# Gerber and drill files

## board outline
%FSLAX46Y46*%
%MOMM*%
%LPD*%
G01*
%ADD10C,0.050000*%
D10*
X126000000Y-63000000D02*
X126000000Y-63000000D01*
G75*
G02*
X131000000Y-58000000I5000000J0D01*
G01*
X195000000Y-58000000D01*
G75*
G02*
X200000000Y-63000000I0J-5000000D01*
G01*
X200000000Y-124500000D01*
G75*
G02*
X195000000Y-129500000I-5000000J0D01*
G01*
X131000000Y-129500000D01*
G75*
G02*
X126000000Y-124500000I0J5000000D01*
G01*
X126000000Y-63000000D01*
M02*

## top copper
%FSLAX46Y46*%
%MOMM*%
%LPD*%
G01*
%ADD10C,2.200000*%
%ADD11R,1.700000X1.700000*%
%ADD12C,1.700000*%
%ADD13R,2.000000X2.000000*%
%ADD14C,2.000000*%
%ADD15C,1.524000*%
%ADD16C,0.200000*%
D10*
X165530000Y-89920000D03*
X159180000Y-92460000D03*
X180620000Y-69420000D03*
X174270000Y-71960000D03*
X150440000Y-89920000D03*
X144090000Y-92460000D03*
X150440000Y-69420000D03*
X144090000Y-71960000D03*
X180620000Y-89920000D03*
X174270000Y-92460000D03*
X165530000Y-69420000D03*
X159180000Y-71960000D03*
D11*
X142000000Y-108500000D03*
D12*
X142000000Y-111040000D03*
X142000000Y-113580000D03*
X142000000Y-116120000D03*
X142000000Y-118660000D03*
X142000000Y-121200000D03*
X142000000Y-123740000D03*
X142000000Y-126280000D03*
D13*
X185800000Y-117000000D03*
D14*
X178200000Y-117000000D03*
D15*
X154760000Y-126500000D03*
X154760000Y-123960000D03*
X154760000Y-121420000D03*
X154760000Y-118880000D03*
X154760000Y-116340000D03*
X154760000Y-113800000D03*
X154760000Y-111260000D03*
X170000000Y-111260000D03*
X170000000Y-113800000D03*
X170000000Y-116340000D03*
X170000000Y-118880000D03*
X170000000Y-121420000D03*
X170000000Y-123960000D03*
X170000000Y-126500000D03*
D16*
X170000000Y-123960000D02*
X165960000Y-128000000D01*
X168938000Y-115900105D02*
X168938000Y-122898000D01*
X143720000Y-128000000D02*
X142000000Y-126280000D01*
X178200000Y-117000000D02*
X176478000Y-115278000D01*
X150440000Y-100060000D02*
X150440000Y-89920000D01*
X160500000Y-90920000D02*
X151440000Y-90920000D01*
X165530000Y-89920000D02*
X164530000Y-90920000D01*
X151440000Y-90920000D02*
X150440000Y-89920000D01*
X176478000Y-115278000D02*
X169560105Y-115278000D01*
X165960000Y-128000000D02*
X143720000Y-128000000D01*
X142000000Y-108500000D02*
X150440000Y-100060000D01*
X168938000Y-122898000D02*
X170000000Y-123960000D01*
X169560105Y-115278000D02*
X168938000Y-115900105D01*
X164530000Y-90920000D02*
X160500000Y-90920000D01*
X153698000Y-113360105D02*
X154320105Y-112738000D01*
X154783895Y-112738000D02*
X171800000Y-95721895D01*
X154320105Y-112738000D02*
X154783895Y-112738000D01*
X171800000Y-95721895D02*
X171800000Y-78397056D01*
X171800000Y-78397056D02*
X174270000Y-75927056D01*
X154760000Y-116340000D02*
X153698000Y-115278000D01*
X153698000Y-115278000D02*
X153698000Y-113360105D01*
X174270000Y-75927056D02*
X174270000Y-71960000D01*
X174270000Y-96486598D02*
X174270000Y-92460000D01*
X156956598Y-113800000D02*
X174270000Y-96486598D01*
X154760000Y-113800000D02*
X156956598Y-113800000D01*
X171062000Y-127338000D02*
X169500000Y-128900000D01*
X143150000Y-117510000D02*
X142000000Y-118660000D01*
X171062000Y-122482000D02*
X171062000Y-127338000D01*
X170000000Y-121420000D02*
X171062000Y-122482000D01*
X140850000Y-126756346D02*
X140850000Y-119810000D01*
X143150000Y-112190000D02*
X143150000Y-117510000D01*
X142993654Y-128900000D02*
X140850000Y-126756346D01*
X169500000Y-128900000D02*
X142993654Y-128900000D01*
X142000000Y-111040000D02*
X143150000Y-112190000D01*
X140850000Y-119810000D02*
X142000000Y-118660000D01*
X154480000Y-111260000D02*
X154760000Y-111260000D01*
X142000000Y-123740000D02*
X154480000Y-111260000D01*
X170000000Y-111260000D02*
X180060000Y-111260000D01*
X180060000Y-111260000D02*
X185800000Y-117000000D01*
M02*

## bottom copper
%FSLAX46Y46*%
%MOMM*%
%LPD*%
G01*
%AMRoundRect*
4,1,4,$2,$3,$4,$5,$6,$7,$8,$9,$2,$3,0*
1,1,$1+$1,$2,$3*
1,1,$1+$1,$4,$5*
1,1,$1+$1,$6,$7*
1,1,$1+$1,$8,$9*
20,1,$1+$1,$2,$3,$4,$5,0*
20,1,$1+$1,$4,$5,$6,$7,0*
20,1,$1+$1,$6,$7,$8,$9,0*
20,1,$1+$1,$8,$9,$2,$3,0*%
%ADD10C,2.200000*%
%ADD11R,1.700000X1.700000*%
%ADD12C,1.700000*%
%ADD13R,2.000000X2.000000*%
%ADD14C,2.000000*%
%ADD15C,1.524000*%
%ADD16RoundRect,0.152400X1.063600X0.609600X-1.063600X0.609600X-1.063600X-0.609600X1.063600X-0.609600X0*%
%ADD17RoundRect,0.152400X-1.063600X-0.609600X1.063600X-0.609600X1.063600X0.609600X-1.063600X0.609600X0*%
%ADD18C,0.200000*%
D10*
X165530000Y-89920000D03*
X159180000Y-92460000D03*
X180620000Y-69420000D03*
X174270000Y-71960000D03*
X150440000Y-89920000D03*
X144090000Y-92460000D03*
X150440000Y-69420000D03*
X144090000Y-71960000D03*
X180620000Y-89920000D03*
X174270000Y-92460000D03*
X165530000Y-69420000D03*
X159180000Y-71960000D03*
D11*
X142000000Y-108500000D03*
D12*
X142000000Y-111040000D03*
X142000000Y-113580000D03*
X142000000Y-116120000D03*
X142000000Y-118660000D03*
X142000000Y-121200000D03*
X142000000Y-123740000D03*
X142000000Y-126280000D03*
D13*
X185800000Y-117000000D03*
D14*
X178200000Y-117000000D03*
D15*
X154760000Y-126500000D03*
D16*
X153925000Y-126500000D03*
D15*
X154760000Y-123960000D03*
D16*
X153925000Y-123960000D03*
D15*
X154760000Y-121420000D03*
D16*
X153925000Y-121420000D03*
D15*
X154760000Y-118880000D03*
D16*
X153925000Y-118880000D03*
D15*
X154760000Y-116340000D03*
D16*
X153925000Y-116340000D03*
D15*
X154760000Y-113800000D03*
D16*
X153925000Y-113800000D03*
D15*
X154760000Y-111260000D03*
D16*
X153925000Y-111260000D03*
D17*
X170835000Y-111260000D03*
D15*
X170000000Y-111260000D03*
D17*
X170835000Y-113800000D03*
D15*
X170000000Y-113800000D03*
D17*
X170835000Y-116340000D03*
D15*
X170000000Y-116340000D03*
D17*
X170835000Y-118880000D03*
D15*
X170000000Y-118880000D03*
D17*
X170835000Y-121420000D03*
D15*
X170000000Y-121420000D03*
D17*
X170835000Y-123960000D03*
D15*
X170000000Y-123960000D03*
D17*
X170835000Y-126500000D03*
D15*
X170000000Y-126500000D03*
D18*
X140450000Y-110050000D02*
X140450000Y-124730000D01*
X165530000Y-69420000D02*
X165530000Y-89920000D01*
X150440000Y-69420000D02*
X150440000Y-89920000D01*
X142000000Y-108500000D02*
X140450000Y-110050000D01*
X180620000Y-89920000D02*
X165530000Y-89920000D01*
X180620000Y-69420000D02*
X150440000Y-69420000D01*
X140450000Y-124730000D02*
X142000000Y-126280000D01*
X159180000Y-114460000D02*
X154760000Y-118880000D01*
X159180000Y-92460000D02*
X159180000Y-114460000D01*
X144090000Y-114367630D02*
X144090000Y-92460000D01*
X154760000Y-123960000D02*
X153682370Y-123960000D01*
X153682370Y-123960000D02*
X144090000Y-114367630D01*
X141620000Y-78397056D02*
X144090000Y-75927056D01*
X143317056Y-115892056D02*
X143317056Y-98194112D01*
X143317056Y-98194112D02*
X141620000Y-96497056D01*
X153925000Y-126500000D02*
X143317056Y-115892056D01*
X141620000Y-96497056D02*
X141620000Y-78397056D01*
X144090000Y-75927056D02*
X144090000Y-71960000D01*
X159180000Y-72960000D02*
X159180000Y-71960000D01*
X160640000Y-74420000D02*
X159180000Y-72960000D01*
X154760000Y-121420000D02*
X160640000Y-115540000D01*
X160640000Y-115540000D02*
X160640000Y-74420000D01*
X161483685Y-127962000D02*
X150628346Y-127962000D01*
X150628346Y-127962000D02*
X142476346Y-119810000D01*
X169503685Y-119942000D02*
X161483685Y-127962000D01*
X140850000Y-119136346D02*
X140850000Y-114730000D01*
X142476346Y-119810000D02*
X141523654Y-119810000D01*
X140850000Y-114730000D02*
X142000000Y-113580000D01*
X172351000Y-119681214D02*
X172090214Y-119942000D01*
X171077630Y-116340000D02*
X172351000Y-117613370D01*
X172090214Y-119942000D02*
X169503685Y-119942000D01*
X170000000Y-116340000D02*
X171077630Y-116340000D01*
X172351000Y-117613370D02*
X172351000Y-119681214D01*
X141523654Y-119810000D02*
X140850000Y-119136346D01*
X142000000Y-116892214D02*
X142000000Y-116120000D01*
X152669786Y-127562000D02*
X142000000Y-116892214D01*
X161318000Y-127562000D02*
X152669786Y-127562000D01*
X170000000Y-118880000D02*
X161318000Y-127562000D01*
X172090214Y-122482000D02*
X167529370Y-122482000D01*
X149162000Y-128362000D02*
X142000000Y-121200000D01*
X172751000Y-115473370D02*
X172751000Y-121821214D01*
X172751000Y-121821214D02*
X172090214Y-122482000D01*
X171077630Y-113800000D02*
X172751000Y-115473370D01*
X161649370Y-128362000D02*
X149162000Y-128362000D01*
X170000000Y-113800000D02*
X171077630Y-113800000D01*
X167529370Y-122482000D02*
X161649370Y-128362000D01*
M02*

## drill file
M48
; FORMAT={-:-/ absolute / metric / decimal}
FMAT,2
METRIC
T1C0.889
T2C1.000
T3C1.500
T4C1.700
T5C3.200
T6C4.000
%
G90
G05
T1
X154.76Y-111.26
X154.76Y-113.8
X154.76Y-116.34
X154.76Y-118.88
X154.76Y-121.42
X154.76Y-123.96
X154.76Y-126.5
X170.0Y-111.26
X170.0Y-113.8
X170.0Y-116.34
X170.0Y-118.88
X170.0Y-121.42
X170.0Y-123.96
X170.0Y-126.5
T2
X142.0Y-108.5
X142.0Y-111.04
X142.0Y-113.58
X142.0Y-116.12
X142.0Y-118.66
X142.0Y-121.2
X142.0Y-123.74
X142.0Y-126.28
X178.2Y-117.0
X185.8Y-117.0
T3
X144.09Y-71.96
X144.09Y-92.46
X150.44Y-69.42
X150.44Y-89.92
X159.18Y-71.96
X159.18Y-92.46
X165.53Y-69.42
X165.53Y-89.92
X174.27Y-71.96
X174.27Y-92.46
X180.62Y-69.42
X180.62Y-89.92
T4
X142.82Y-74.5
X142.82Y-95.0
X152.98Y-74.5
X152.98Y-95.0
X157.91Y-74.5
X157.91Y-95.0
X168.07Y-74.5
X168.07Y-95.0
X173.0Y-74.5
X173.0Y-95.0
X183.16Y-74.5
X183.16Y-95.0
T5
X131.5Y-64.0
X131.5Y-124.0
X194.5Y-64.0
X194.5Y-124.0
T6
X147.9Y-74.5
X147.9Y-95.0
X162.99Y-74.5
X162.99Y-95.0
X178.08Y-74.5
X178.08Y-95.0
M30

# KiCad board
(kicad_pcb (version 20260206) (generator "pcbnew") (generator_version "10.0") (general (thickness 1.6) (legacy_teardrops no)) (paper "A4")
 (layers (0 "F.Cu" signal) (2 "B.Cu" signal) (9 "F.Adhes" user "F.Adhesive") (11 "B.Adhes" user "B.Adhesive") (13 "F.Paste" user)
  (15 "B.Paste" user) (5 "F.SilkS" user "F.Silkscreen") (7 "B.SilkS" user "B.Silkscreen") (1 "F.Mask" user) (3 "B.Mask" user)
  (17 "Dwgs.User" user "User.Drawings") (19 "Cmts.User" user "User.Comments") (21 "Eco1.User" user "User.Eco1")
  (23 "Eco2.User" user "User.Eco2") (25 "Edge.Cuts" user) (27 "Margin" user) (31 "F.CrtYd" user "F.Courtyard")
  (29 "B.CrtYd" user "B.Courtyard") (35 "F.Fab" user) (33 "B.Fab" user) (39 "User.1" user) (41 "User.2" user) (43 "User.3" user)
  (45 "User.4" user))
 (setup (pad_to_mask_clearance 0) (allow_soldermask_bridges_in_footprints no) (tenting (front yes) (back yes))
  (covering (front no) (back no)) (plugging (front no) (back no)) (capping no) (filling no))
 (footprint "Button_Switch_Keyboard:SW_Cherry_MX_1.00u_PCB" (layer "F.Cu") (at 165.53 89.92)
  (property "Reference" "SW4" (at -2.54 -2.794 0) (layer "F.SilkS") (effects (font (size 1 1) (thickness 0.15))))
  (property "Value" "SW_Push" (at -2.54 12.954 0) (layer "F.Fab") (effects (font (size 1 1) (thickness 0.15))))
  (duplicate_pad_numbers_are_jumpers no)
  (pad "" np_thru_hole circle (at -7.62 5.08) (size 1.7 1.7) (drill 1.7) (layers "*.Cu" "*.Mask"))
  (pad "" np_thru_hole circle (at -2.54 5.08) (size 4 4) (drill 4) (layers "*.Cu" "*.Mask"))
  (pad "" np_thru_hole circle (at 2.54 5.08) (size 1.7 1.7) (drill 1.7) (layers "*.Cu" "*.Mask"))
  (pad "1" thru_hole circle (at 0 0) (size 2.2 2.2) (drill 1.5) (layers "*.Cu" "*.Mask") (remove_unused_layers no) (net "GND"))
  (pad "2" thru_hole circle (at -6.35 2.54) (size 2.2 2.2) (drill 1.5) (layers "*.Cu" "*.Mask") (remove_unused_layers no)
   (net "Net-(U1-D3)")))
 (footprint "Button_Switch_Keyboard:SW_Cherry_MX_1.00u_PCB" (layer "F.Cu") (at 180.62 69.42)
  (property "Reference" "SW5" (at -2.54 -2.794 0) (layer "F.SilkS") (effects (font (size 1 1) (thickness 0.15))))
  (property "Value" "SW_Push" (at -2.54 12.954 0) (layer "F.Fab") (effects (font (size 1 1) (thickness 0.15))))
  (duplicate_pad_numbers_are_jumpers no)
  (pad "" np_thru_hole circle (at -7.62 5.08) (size 1.7 1.7) (drill 1.7) (layers "*.Cu" "*.Mask"))
  (pad "" np_thru_hole circle (at -2.54 5.08) (size 4 4) (drill 4) (layers "*.Cu" "*.Mask"))
  (pad "" np_thru_hole circle (at 2.54 5.08) (size 1.7 1.7) (drill 1.7) (layers "*.Cu" "*.Mask"))
  (pad "1" thru_hole circle (at 0 0) (size 2.2 2.2) (drill 1.5) (layers "*.Cu" "*.Mask") (remove_unused_layers no) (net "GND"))
  (pad "2" thru_hole circle (at -6.35 2.54) (size 2.2 2.2) (drill 1.5) (layers "*.Cu" "*.Mask") (remove_unused_layers no)
   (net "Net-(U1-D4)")))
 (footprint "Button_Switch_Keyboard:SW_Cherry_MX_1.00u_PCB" (layer "F.Cu") (at 150.44 89.92)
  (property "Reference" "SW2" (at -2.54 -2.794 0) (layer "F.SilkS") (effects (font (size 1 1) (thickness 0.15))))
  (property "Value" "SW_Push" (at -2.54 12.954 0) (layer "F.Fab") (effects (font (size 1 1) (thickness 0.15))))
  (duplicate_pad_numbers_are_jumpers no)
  (pad "" np_thru_hole circle (at -7.62 5.08) (size 1.7 1.7) (drill 1.7) (layers "*.Cu" "*.Mask"))
  (pad "" np_thru_hole circle (at -2.54 5.08) (size 4 4) (drill 4) (layers "*.Cu" "*.Mask"))
  (pad "" np_thru_hole circle (at 2.54 5.08) (size 1.7 1.7) (drill 1.7) (layers "*.Cu" "*.Mask"))
  (pad "1" thru_hole circle (at 0 0) (size 2.2 2.2) (drill 1.5) (layers "*.Cu" "*.Mask") (remove_unused_layers no) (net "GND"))
  (pad "2" thru_hole circle (at -6.35 2.54) (size 2.2 2.2) (drill 1.5) (layers "*.Cu" "*.Mask") (remove_unused_layers no)
   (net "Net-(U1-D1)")))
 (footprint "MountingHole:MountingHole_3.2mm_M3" (layer "F.Cu") (at 131.5 64)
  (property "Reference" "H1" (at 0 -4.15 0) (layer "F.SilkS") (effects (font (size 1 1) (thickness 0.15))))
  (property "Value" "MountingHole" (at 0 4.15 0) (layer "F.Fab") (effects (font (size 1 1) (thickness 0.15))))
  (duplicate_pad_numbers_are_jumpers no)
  (pad "" np_thru_hole circle (at 0 0) (size 3.2 3.2) (drill 3.2) (layers "*.Cu" "*.Mask")))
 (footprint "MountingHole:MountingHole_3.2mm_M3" (layer "F.Cu") (at 194.5 64)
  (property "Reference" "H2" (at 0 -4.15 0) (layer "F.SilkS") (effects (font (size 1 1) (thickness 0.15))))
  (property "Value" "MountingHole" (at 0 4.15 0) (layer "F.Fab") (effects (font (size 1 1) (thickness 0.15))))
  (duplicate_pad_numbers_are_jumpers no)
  (pad "" np_thru_hole circle (at 0 0) (size 3.2 3.2) (drill 3.2) (layers "*.Cu" "*.Mask")))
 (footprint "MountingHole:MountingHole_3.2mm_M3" (layer "F.Cu") (at 131.5 124)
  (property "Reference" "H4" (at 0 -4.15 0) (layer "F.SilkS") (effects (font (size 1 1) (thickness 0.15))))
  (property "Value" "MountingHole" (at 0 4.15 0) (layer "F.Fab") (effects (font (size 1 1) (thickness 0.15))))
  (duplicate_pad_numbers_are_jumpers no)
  (pad "" np_thru_hole circle (at 0 0) (size 3.2 3.2) (drill 3.2) (layers "*.Cu" "*.Mask")))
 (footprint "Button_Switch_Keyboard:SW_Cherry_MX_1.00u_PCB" (layer "F.Cu") (at 150.44 69.42)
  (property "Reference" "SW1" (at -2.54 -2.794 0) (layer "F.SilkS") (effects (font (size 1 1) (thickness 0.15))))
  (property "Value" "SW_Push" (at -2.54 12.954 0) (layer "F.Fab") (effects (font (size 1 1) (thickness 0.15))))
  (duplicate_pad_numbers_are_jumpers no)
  (pad "" np_thru_hole circle (at -7.62 5.08) (size 1.7 1.7) (drill 1.7) (layers "*.Cu" "*.Mask"))
  (pad "" np_thru_hole circle (at -2.54 5.08) (size 4 4) (drill 4) (layers "*.Cu" "*.Mask"))
  (pad "" np_thru_hole circle (at 2.54 5.08) (size 1.7 1.7) (drill 1.7) (layers "*.Cu" "*.Mask"))
  (pad "1" thru_hole circle (at 0 0) (size 2.2 2.2) (drill 1.5) (layers "*.Cu" "*.Mask") (remove_unused_layers no) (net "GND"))
  (pad "2" thru_hole circle (at -6.35 2.54) (size 2.2 2.2) (drill 1.5) (layers "*.Cu" "*.Mask") (remove_unused_layers no)
   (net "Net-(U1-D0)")))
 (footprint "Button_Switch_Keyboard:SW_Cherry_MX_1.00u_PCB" (layer "F.Cu") (at 180.62 89.92)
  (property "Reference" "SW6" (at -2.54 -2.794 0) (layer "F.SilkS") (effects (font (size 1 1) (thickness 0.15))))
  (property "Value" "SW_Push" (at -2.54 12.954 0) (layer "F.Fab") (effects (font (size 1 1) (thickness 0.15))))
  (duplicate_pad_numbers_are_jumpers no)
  (pad "" np_thru_hole circle (at -7.62 5.08) (size 1.7 1.7) (drill 1.7) (layers "*.Cu" "*.Mask"))
  (pad "" np_thru_hole circle (at -2.54 5.08) (size 4 4) (drill 4) (layers "*.Cu" "*.Mask"))
  (pad "" np_thru_hole circle (at 2.54 5.08) (size 1.7 1.7) (drill 1.7) (layers "*.Cu" "*.Mask"))
  (pad "1" thru_hole circle (at 0 0) (size 2.2 2.2) (drill 1.5) (layers "*.Cu" "*.Mask") (remove_unused_layers no) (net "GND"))
  (pad "2" thru_hole circle (at -6.35 2.54) (size 2.2 2.2) (drill 1.5) (layers "*.Cu" "*.Mask") (remove_unused_layers no)
   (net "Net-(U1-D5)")))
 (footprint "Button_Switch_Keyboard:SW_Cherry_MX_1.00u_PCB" (layer "F.Cu") (at 165.53 69.42)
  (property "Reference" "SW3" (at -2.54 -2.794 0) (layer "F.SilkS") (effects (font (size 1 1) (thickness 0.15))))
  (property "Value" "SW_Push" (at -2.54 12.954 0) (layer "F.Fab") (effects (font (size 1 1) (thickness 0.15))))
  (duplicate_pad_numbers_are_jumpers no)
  (pad "" np_thru_hole circle (at -7.62 5.08) (size 1.7 1.7) (drill 1.7) (layers "*.Cu" "*.Mask"))
  (pad "" np_thru_hole circle (at -2.54 5.08) (size 4 4) (drill 4) (layers "*.Cu" "*.Mask"))
  (pad "" np_thru_hole circle (at 2.54 5.08) (size 1.7 1.7) (drill 1.7) (layers "*.Cu" "*.Mask"))
  (pad "1" thru_hole circle (at 0 0) (size 2.2 2.2) (drill 1.5) (layers "*.Cu" "*.Mask") (remove_unused_layers no) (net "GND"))
  (pad "2" thru_hole circle (at -6.35 2.54) (size 2.2 2.2) (drill 1.5) (layers "*.Cu" "*.Mask") (remove_unused_layers no)
   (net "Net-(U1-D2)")))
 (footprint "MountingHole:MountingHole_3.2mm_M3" (layer "F.Cu") (at 194.5 124)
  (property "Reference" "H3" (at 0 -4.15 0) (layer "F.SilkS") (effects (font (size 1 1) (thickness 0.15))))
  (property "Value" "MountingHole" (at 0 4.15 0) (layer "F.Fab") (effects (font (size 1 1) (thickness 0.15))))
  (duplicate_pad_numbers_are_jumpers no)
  (pad "" np_thru_hole circle (at 0 0) (size 3.2 3.2) (drill 3.2) (layers "*.Cu" "*.Mask")))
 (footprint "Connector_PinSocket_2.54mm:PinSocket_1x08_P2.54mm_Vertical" (layer "B.Cu") (at 142 108.5 180)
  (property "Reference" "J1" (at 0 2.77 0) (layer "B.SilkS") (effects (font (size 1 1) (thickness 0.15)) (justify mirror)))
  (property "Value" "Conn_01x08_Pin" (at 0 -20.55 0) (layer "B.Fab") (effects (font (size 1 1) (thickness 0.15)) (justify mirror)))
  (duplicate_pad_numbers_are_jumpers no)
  (pad "1" thru_hole rect (at 0 0 180) (size 1.7 1.7) (drill 1) (layers "*.Cu" "*.Mask") (remove_unused_layers no) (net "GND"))
  (pad "2" thru_hole circle (at 0 -2.54 180) (size 1.7 1.7) (drill 1) (layers "*.Cu" "*.Mask") (remove_unused_layers no) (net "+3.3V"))
  (pad "3" thru_hole circle (at 0 -5.08 180) (size 1.7 1.7) (drill 1) (layers "*.Cu" "*.Mask") (remove_unused_layers no) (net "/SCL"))
  (pad "4" thru_hole circle (at 0 -7.62 180) (size 1.7 1.7) (drill 1) (layers "*.Cu" "*.Mask") (remove_unused_layers no) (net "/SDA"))
  (pad "5" thru_hole circle (at 0 -10.16 180) (size 1.7 1.7) (drill 1) (layers "*.Cu" "*.Mask") (remove_unused_layers no) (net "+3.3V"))
  (pad "6" thru_hole circle (at 0 -12.7 180) (size 1.7 1.7) (drill 1) (layers "*.Cu" "*.Mask") (remove_unused_layers no) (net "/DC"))
  (pad "7" thru_hole circle (at 0 -15.24 180) (size 1.7 1.7) (drill 1) (layers "*.Cu" "*.Mask") (remove_unused_layers no) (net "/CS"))
  (pad "8" thru_hole circle (at 0 -17.78 180) (size 1.7 1.7) (drill 1) (layers "*.Cu" "*.Mask") (remove_unused_layers no) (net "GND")))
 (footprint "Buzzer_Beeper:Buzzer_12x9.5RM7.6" (layer "B.Cu") (at 185.8 117 180)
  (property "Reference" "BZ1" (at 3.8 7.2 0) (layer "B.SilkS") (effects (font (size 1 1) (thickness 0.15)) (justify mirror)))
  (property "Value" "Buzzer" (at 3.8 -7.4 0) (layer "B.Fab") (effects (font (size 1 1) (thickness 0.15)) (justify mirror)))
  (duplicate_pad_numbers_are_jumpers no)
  (pad "1" thru_hole rect (at 0 0 180) (size 2 2) (drill 1) (layers "*.Cu" "*.Mask") (remove_unused_layers no) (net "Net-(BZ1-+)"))
  (pad "2" thru_hole circle (at 7.6 0 180) (size 2 2) (drill 1) (layers "*.Cu" "*.Mask") (remove_unused_layers no) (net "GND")))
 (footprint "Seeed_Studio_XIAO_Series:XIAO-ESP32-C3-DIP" (layer "B.Cu") (at 162.38 118.88 -90)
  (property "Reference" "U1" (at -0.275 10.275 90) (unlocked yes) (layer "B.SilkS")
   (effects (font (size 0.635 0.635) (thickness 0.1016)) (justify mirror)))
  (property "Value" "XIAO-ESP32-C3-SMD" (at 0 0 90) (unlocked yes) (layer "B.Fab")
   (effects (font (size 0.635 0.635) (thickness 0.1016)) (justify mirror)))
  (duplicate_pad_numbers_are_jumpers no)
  (pad "1" thru_hole circle (at 7.62 7.62 180) (size 1.524 1.524) (drill 0.889) (layers "*.Cu" "*.Mask") (remove_unused_layers no)
   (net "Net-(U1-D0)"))
  (pad "1" smd roundrect (at 7.62 8.455 180) (size 2.432 1.524) (layers "B.Cu" "B.Mask") (roundrect_rratio 0.1) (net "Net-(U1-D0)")
   (thermal_bridge_angle 45))
  (pad "2" thru_hole circle (at 5.08 7.62 180) (size 1.524 1.524) (drill 0.889) (layers "*.Cu" "*.Mask") (remove_unused_layers no)
   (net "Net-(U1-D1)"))
  (pad "2" smd roundrect (at 5.08 8.455 180) (size 2.432 1.524) (layers "B.Cu" "B.Mask") (roundrect_rratio 0.1) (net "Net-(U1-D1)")
   (thermal_bridge_angle 45))
  (pad "3" thru_hole circle (at 2.54 7.62 180) (size 1.524 1.524) (drill 0.889) (layers "*.Cu" "*.Mask") (remove_unused_layers no)
   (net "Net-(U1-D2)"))
  (pad "3" smd roundrect (at 2.54 8.455 180) (size 2.432 1.524) (layers "B.Cu" "B.Mask") (roundrect_rratio 0.1) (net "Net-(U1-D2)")
   (thermal_bridge_angle 45))
  (pad "4" thru_hole circle (at 0 7.62 180) (size 1.524 1.524) (drill 0.889) (layers "*.Cu" "*.Mask") (remove_unused_layers no)
   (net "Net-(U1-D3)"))
  (pad "4" smd roundrect (at 0 8.455 180) (size 2.432 1.524) (layers "B.Cu" "B.Mask") (roundrect_rratio 0.1) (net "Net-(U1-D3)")
   (thermal_bridge_angle 45))
  (pad "5" thru_hole circle (at -2.54 7.62 180) (size 1.524 1.524) (drill 0.889) (layers "*.Cu" "*.Mask") (remove_unused_layers no)
   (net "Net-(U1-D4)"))
  (pad "5" smd roundrect (at -2.54 8.455 180) (size 2.432 1.524) (layers "B.Cu" "B.Mask") (roundrect_rratio 0.1) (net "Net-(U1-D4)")
   (thermal_bridge_angle 45))
  (pad "6" thru_hole circle (at -5.08 7.62 180) (size 1.524 1.524) (drill 0.889) (layers "*.Cu" "*.Mask") (remove_unused_layers no)
   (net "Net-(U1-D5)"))
  (pad "6" smd roundrect (at -5.08 8.455 180) (size 2.432 1.524) (layers "B.Cu" "B.Mask") (roundrect_rratio 0.1) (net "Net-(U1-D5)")
   (thermal_bridge_angle 45))
  (pad "7" thru_hole circle (at -7.62 7.62 180) (size 1.524 1.524) (drill 0.889) (layers "*.Cu" "*.Mask") (remove_unused_layers no)
   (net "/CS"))
  (pad "7" smd roundrect (at -7.62 8.455 180) (size 2.432 1.524) (layers "B.Cu" "B.Mask") (roundrect_rratio 0.1) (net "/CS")
   (thermal_bridge_angle 45))
  (pad "8" smd roundrect (at -7.62 -8.455) (size 2.432 1.524) (layers "B.Cu" "B.Mask") (roundrect_rratio 0.1) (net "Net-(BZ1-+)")
   (thermal_bridge_angle 45))
  (pad "8" thru_hole circle (at -7.62 -7.62) (size 1.524 1.524) (drill 0.889) (layers "*.Cu" "*.Mask") (remove_unused_layers no)
   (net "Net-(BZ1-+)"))
  (pad "9" smd roundrect (at -5.08 -8.455) (size 2.432 1.524) (layers "B.Cu" "B.Mask") (roundrect_rratio 0.1) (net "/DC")
   (thermal_bridge_angle 45))
  (pad "9" thru_hole circle (at -5.08 -7.62) (size 1.524 1.524) (drill 0.889) (layers "*.Cu" "*.Mask") (remove_unused_layers no) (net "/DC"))
  (pad "10" smd roundrect (at -2.54 -8.455) (size 2.432 1.524) (layers "B.Cu" "B.Mask") (roundrect_rratio 0.1) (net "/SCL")
   (thermal_bridge_angle 45))
  (pad "10" thru_hole circle (at -2.54 -7.62) (size 1.524 1.524) (drill 0.889) (layers "*.Cu" "*.Mask") (remove_unused_layers no)
   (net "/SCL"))
  (pad "11" smd roundrect (at 0 -8.455) (size 2.432 1.524) (layers "B.Cu" "B.Mask") (roundrect_rratio 0.1) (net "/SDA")
   (thermal_bridge_angle 45))
  (pad "11" thru_hole circle (at 0 -7.62) (size 1.524 1.524) (drill 0.889) (layers "*.Cu" "*.Mask") (remove_unused_layers no) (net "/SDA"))
  (pad "12" smd roundrect (at 2.54 -8.455) (size 2.432 1.524) (layers "B.Cu" "B.Mask") (roundrect_rratio 0.1) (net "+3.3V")
   (thermal_bridge_angle 45))
  (pad "12" thru_hole circle (at 2.54 -7.62) (size 1.524 1.524) (drill 0.889) (layers "*.Cu" "*.Mask") (remove_unused_layers no)
   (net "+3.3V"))
  (pad "13" smd roundrect (at 5.08 -8.455) (size 2.432 1.524) (layers "B.Cu" "B.Mask") (roundrect_rratio 0.1) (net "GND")
   (thermal_bridge_angle 45))
  (pad "13" thru_hole circle (at 5.08 -7.62) (size 1.524 1.524) (drill 0.889) (layers "*.Cu" "*.Mask") (remove_unused_layers no) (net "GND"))
  (pad "14" smd roundrect (at 7.62 -8.455) (size 2.432 1.524) (layers "B.Cu" "B.Mask") (roundrect_rratio 0.1)
   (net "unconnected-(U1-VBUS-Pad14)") (thermal_bridge_angle 45))
  (pad "14" thru_hole circle (at 7.62 -7.62) (size 1.524 1.524) (drill 0.889) (layers "*.Cu" "*.Mask") (remove_unused_layers no)
   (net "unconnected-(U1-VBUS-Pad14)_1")))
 (gr_rect (start 126 58) (end 200 129.5) (radius 5) (stroke (width 0.05) (type solid)) (fill no) (layer "Edge.Cuts"))
 (segment (start 170 123.96) (end 165.96 128) (width 0.2) (layer "F.Cu") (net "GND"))
 (segment (start 168.938 115.900105) (end 168.938 122.898) (width 0.2) (layer "F.Cu") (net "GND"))
 (segment (start 143.72 128) (end 142 126.28) (width 0.2) (layer "F.Cu") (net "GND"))
 (segment (start 178.2 117) (end 176.478 115.278) (width 0.2) (layer "F.Cu") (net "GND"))
 (segment (start 150.44 100.06) (end 150.44 89.92) (width 0.2) (layer "F.Cu") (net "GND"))
 (segment (start 160.5 90.92) (end 151.44 90.92) (width 0.2) (layer "F.Cu") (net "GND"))
 (segment (start 165.53 89.92) (end 164.53 90.92) (width 0.2) (layer "F.Cu") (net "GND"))
 (segment (start 151.44 90.92) (end 150.44 89.92) (width 0.2) (layer "F.Cu") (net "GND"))
 (segment (start 176.478 115.278) (end 169.560105 115.278) (width 0.2) (layer "F.Cu") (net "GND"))
 (segment (start 165.96 128) (end 143.72 128) (width 0.2) (layer "F.Cu") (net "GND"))
 (segment (start 142 108.5) (end 150.44 100.06) (width 0.2) (layer "F.Cu") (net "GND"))
 (segment (start 168.938 122.898) (end 170 123.96) (width 0.2) (layer "F.Cu") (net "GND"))
 (segment (start 169.560105 115.278) (end 168.938 115.900105) (width 0.2) (layer "F.Cu") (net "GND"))
 (segment (start 164.53 90.92) (end 160.5 90.92) (width 0.2) (layer "F.Cu") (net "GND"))
 (segment (start 140.45 110.05) (end 140.45 124.73) (width 0.2) (layer "B.Cu") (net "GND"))
 (segment (start 165.53 69.42) (end 165.53 89.92) (width 0.2) (layer "B.Cu") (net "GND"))
 (segment (start 150.44 69.42) (end 150.44 89.92) (width 0.2) (layer "B.Cu") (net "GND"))
 (segment (start 142 108.5) (end 140.45 110.05) (width 0.2) (layer "B.Cu") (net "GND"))
 (segment (start 180.62 89.92) (end 165.53 89.92) (width 0.2) (layer "B.Cu") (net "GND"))
 (segment (start 180.62 69.42) (end 150.44 69.42) (width 0.2) (layer "B.Cu") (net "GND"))
 (segment (start 140.45 124.73) (end 142 126.28) (width 0.2) (layer "B.Cu") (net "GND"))
 (segment (start 159.18 114.46) (end 154.76 118.88) (width 0.2) (layer "B.Cu") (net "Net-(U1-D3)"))
 (segment (start 159.18 92.46) (end 159.18 114.46) (width 0.2) (layer "B.Cu") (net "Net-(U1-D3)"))
 (segment (start 153.698 113.360105) (end 154.320105 112.738) (width 0.2) (layer "F.Cu") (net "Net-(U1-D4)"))
 (segment (start 154.783895 112.738) (end 171.8 95.721895) (width 0.2) (layer "F.Cu") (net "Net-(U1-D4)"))
 (segment (start 154.320105 112.738) (end 154.783895 112.738) (width 0.2) (layer "F.Cu") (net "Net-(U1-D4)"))
 (segment (start 171.8 95.721895) (end 171.8 78.397056) (width 0.2) (layer "F.Cu") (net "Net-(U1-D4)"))
 (segment (start 171.8 78.397056) (end 174.27 75.927056) (width 0.2) (layer "F.Cu") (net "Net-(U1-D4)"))
 (segment (start 154.76 116.34) (end 153.698 115.278) (width 0.2) (layer "F.Cu") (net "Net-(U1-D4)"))
 (segment (start 153.698 115.278) (end 153.698 113.360105) (width 0.2) (layer "F.Cu") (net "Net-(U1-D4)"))
 (segment (start 174.27 75.927056) (end 174.27 71.96) (width 0.2) (layer "F.Cu") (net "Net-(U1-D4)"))
 (segment (start 144.09 114.36763) (end 144.09 92.46) (width 0.2) (layer "B.Cu") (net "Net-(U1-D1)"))
 (segment (start 154.76 123.96) (end 153.68237 123.96) (width 0.2) (layer "B.Cu") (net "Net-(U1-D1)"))
 (segment (start 153.68237 123.96) (end 144.09 114.36763) (width 0.2) (layer "B.Cu") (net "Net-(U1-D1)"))
 (segment (start 141.62 78.397056) (end 144.09 75.927056) (width 0.2) (layer "B.Cu") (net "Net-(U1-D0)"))
 (segment (start 143.317056 115.892056) (end 143.317056 98.194112) (width 0.2) (layer "B.Cu") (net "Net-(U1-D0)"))
 (segment (start 143.317056 98.194112) (end 141.62 96.497056) (width 0.2) (layer "B.Cu") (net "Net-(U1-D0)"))
 (segment (start 153.925 126.5) (end 143.317056 115.892056) (width 0.2) (layer "B.Cu") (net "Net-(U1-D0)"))
 (segment (start 141.62 96.497056) (end 141.62 78.397056) (width 0.2) (layer "B.Cu") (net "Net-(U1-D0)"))
 (segment (start 144.09 75.927056) (end 144.09 71.96) (width 0.2) (layer "B.Cu") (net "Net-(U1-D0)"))
 (segment (start 174.27 96.486598) (end 174.27 92.46) (width 0.2) (layer "F.Cu") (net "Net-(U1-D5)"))
 (segment (start 156.956598 113.8) (end 174.27 96.486598) (width 0.2) (layer "F.Cu") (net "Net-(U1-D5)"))
 (segment (start 154.76 113.8) (end 156.956598 113.8) (width 0.2) (layer "F.Cu") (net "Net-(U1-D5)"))
 (segment (start 159.18 72.96) (end 159.18 71.96) (width 0.2) (layer "B.Cu") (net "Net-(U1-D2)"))
 (segment (start 160.64 74.42) (end 159.18 72.96) (width 0.2) (layer "B.Cu") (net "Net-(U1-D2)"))
 (segment (start 154.76 121.42) (end 160.64 115.54) (width 0.2) (layer "B.Cu") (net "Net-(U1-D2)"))
 (segment (start 160.64 115.54) (end 160.64 74.42) (width 0.2) (layer "B.Cu") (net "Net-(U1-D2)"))
 (segment (start 171.062 127.338) (end 169.5 128.9) (width 0.2) (layer "F.Cu") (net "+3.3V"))
 (segment (start 143.15 117.51) (end 142 118.66) (width 0.2) (layer "F.Cu") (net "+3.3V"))
 (segment (start 171.062 122.482) (end 171.062 127.338) (width 0.2) (layer "F.Cu") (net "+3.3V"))
 (segment (start 170 121.42) (end 171.062 122.482) (width 0.2) (layer "F.Cu") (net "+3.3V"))
 (segment (start 140.85 126.756346) (end 140.85 119.81) (width 0.2) (layer "F.Cu") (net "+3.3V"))
 (segment (start 143.15 112.19) (end 143.15 117.51) (width 0.2) (layer "F.Cu") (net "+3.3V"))
 (segment (start 142.993654 128.9) (end 140.85 126.756346) (width 0.2) (layer "F.Cu") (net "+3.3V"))
 (segment (start 169.5 128.9) (end 142.993654 128.9) (width 0.2) (layer "F.Cu") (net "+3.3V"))
 (segment (start 142 111.04) (end 143.15 112.19) (width 0.2) (layer "F.Cu") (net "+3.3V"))
 (segment (start 140.85 119.81) (end 142 118.66) (width 0.2) (layer "F.Cu") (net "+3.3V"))
 (segment (start 161.483685 127.962) (end 150.628346 127.962) (width 0.2) (layer "B.Cu") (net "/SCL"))
 (segment (start 150.628346 127.962) (end 142.476346 119.81) (width 0.2) (layer "B.Cu") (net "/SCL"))
 (segment (start 169.503685 119.942) (end 161.483685 127.962) (width 0.2) (layer "B.Cu") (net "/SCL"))
 (segment (start 140.85 119.136346) (end 140.85 114.73) (width 0.2) (layer "B.Cu") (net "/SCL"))
 (segment (start 142.476346 119.81) (end 141.523654 119.81) (width 0.2) (layer "B.Cu") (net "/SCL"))
 (segment (start 140.85 114.73) (end 142 113.58) (width 0.2) (layer "B.Cu") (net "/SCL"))
 (segment (start 172.351 119.681214) (end 172.090214 119.942) (width 0.2) (layer "B.Cu") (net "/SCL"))
 (segment (start 171.07763 116.34) (end 172.351 117.61337) (width 0.2) (layer "B.Cu") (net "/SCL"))
 (segment (start 172.090214 119.942) (end 169.503685 119.942) (width 0.2) (layer "B.Cu") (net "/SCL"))
 (segment (start 170 116.34) (end 171.07763 116.34) (width 0.2) (layer "B.Cu") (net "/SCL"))
 (segment (start 172.351 117.61337) (end 172.351 119.681214) (width 0.2) (layer "B.Cu") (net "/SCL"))
 (segment (start 141.523654 119.81) (end 140.85 119.136346) (width 0.2) (layer "B.Cu") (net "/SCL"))
 (segment (start 142 116.892214) (end 142 116.12) (width 0.2) (layer "B.Cu") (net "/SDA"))
 (segment (start 152.669786 127.562) (end 142 116.892214) (width 0.2) (layer "B.Cu") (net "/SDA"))
 (segment (start 161.318 127.562) (end 152.669786 127.562) (width 0.2) (layer "B.Cu") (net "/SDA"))
 (segment (start 170 118.88) (end 161.318 127.562) (width 0.2) (layer "B.Cu") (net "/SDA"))
 (segment (start 172.090214 122.482) (end 167.52937 122.482) (width 0.2) (layer "B.Cu") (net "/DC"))
 (segment (start 149.162 128.362) (end 142 121.2) (width 0.2) (layer "B.Cu") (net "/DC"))
 (segment (start 172.751 115.47337) (end 172.751 121.821214) (width 0.2) (layer "B.Cu") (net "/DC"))
 (segment (start 172.751 121.821214) (end 172.090214 122.482) (width 0.2) (layer "B.Cu") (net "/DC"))
 (segment (start 171.07763 113.8) (end 172.751 115.47337) (width 0.2) (layer "B.Cu") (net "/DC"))
 (segment (start 161.64937 128.362) (end 149.162 128.362) (width 0.2) (layer "B.Cu") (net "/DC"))
 (segment (start 170 113.8) (end 171.07763 113.8) (width 0.2) (layer "B.Cu") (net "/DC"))
 (segment (start 167.52937 122.482) (end 161.64937 128.362) (width 0.2) (layer "B.Cu") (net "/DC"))
 (segment (start 154.48 111.26) (end 154.76 111.26) (width 0.2) (layer "F.Cu") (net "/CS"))
 (segment (start 142 123.74) (end 154.48 111.26) (width 0.2) (layer "F.Cu") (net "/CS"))
 (segment (start 170 111.26) (end 180.06 111.26) (width 0.2) (layer "F.Cu") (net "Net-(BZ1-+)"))
 (segment (start 180.06 111.26) (end 185.8 117) (width 0.2) (layer "F.Cu") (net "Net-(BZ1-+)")))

